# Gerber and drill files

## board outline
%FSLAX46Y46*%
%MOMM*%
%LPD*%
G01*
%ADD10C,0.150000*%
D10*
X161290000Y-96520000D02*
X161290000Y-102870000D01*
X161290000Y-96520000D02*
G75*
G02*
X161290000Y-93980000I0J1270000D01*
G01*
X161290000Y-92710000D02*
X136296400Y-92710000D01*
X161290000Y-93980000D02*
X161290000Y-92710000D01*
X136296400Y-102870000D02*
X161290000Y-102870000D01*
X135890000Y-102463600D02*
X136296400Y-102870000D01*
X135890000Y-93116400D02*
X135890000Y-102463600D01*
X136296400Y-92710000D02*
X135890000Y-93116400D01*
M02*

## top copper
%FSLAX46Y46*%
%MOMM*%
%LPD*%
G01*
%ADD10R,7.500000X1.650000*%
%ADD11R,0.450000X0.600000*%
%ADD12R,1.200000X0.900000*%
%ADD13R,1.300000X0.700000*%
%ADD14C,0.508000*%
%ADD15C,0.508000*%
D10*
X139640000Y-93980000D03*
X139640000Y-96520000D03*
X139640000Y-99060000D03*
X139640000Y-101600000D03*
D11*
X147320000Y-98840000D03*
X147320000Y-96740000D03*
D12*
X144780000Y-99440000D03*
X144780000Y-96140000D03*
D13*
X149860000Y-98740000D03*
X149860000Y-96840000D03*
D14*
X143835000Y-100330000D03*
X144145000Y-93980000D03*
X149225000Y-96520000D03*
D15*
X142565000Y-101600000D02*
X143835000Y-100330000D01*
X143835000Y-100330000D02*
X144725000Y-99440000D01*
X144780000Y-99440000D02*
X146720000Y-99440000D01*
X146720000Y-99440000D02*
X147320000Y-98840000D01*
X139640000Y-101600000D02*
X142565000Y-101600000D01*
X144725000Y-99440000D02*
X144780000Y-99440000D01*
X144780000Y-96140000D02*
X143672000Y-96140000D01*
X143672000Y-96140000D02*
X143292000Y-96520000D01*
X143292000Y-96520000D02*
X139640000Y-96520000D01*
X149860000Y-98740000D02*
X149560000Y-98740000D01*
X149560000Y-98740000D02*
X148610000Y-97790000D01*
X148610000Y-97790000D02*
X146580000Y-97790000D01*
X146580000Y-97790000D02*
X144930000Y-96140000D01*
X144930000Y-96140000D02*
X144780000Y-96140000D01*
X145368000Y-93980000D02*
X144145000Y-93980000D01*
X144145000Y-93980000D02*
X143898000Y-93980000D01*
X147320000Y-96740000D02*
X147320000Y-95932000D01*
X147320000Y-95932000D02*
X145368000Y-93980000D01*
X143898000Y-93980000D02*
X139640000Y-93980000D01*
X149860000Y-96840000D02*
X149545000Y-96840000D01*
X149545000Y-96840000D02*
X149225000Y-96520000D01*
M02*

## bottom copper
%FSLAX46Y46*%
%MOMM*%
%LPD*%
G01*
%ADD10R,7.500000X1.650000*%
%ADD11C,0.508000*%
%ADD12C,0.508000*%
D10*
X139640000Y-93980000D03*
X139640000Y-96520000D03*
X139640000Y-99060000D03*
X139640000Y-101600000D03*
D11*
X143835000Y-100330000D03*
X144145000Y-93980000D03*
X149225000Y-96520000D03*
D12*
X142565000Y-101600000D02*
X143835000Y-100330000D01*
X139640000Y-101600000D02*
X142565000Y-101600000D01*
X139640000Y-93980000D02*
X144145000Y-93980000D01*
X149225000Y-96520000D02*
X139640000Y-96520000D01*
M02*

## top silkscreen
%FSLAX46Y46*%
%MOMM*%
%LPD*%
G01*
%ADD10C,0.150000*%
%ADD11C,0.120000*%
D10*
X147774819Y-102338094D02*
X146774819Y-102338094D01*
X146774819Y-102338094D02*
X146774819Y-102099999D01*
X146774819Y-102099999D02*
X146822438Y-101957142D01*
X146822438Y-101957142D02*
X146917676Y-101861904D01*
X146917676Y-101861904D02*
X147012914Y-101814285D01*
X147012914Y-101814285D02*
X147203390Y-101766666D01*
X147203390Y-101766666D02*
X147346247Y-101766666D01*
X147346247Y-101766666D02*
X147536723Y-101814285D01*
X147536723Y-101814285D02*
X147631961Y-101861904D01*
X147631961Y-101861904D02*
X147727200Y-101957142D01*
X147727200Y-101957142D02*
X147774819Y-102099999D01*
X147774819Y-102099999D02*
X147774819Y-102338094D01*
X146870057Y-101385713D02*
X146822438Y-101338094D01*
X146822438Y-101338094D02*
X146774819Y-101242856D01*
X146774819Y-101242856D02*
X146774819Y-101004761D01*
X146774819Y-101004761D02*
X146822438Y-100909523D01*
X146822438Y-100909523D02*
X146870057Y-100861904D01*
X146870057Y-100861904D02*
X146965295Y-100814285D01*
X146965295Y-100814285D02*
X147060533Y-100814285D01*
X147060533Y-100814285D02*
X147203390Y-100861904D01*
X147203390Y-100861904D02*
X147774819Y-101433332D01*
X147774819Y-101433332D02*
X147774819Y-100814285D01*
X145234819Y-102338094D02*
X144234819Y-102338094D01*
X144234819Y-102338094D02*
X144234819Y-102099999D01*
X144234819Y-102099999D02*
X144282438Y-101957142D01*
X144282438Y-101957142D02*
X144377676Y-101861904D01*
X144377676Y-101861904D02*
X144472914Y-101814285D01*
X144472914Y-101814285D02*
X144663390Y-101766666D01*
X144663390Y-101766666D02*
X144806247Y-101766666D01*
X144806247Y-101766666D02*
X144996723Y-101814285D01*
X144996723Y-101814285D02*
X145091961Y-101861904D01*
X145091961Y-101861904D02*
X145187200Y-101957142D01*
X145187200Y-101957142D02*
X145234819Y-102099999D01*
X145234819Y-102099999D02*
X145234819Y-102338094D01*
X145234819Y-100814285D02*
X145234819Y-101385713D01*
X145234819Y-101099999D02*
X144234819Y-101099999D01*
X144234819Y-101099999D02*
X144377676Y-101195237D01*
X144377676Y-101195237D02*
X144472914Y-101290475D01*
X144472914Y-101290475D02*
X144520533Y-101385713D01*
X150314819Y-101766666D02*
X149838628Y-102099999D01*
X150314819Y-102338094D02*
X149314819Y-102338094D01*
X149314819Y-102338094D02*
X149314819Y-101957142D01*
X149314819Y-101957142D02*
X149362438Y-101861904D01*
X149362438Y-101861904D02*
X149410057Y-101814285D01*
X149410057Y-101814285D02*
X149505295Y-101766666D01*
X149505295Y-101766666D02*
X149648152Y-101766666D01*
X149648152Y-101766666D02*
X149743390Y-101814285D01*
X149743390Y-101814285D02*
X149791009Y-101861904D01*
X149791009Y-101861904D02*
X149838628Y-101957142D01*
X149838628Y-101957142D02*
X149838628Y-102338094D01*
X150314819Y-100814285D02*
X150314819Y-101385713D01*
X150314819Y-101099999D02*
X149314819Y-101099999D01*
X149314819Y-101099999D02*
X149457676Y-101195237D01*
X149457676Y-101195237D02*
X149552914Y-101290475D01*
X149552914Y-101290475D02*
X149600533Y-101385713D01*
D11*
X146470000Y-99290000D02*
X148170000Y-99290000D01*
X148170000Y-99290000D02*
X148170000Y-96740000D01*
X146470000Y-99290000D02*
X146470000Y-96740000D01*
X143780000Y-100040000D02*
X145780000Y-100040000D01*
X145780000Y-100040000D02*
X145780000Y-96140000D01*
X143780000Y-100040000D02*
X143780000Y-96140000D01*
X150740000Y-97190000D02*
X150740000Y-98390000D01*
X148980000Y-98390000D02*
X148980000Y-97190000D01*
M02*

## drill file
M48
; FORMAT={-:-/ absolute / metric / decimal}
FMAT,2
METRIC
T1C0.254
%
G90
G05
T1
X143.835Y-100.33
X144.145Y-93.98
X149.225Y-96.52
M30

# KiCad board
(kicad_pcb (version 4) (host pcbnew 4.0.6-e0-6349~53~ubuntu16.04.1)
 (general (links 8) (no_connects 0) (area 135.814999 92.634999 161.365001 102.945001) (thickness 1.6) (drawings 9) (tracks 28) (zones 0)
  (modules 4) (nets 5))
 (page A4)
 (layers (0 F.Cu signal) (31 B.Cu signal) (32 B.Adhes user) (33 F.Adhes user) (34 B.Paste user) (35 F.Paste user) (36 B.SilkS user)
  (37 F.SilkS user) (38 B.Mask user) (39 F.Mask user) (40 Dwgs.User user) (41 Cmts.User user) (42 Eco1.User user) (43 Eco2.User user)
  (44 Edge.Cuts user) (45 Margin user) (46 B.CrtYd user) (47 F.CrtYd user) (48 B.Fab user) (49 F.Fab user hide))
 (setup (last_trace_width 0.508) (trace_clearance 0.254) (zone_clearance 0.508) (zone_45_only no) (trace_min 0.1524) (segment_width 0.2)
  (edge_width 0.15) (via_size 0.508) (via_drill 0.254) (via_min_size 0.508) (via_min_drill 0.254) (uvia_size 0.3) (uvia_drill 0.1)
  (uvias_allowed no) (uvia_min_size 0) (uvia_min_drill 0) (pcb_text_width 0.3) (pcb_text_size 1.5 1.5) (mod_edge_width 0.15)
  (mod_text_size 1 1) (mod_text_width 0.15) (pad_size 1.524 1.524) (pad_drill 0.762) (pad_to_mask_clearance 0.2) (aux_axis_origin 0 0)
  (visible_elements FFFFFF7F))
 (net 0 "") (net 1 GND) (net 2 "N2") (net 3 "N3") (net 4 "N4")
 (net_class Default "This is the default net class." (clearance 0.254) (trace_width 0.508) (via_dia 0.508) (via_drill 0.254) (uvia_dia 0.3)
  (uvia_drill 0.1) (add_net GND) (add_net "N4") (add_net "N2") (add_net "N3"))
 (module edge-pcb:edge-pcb (layer F.Cu) (at 135.89 97.79 270)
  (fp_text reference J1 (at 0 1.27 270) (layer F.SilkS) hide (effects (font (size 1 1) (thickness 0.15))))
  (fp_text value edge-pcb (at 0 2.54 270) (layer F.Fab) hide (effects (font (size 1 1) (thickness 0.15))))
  (pad 1 smd rect (at -3.81 -3.75 270) (size 1.65 7.5) (layers F.Cu F.Paste F.Mask) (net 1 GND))
  (pad 2 smd rect (at -3.81 -3.75 270) (size 1.65 7.5) (layers B.Cu B.Paste B.Mask) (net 1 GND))
  (pad 3 smd rect (at -1.27 -3.75 270) (size 1.65 7.5) (layers F.Cu F.Paste F.Mask) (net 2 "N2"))
  (pad 4 smd rect (at -1.27 -3.75 270) (size 1.65 7.5) (layers B.Cu B.Paste B.Mask) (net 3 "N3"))
  (pad 5 smd rect (at 1.27 -3.75 270) (size 1.65 7.5) (layers F.Cu F.Paste F.Mask))
  (pad 6 smd rect (at 1.27 -3.75 270) (size 1.65 7.5) (layers B.Cu B.Paste B.Mask))
  (pad 7 smd rect (at 3.81 -3.75 270) (size 1.65 7.5) (layers F.Cu F.Paste F.Mask) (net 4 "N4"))
  (pad 8 smd rect (at 3.81 -3.75 270) (size 1.65 7.5) (layers B.Cu B.Paste B.Mask) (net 4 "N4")))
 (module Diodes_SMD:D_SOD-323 (layer F.Cu) (at 147.32 97.79 90)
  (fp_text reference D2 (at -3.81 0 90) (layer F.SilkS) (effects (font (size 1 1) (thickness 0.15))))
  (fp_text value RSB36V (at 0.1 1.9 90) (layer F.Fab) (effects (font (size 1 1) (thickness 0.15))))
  (fp_line (start -1.5 -0.85) (end -1.5 0.85) (layer F.SilkS) (width 0.12))
  (fp_line (start -1.5 0.85) (end 1.05 0.85) (layer F.SilkS) (width 0.12))
  (fp_line (start -1.5 -0.85) (end 1.05 -0.85) (layer F.SilkS) (width 0.12))
  (pad 1 smd rect (at -1.05 0 90) (size 0.6 0.45) (layers F.Cu F.Paste F.Mask) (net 4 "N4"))
  (pad 2 smd rect (at 1.05 0 90) (size 0.6 0.45) (layers F.Cu F.Paste F.Mask) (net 1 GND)))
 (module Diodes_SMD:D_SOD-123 (layer F.Cu) (at 144.78 97.79 90)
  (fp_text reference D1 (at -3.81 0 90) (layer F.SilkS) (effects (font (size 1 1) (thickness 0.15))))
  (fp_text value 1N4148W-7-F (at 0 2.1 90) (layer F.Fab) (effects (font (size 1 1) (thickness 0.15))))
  (fp_line (start -2.25 -1) (end -2.25 1) (layer F.SilkS) (width 0.12))
  (fp_line (start -2.25 1) (end 1.65 1) (layer F.SilkS) (width 0.12))
  (fp_line (start -2.25 -1) (end 1.65 -1) (layer F.SilkS) (width 0.12))
  (pad 1 smd rect (at -1.65 0 90) (size 0.9 1.2) (layers F.Cu F.Paste F.Mask) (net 4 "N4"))
  (pad 2 smd rect (at 1.65 0 90) (size 0.9 1.2) (layers F.Cu F.Paste F.Mask) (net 2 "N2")))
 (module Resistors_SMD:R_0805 (layer F.Cu) (at 149.86 97.79 90)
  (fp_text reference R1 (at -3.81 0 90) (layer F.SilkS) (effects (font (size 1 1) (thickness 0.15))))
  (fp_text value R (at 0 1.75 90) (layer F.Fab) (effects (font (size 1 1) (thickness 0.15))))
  (fp_line (start 0.6 0.88) (end -0.6 0.88) (layer F.SilkS) (width 0.12))
  (fp_line (start -0.6 -0.88) (end 0.6 -0.88) (layer F.SilkS) (width 0.12))
  (pad 1 smd rect (at -0.95 0 90) (size 0.7 1.3) (layers F.Cu F.Paste F.Mask) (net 2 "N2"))
  (pad 2 smd rect (at 0.95 0 90) (size 0.7 1.3) (layers F.Cu F.Paste F.Mask) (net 3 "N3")))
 (gr_line (start 161.29 96.52) (end 161.29 102.87) (layer Edge.Cuts) (width 0.15))
 (gr_arc (start 161.29 95.25) (end 161.29 96.52) (angle 180) (layer Edge.Cuts) (width 0.15))
 (gr_line (start 161.29 92.71) (end 136.2964 92.71) (layer Edge.Cuts) (width 0.15))
 (gr_line (start 161.29 93.98) (end 161.29 92.71) (layer Edge.Cuts) (width 0.15))
 (gr_line (start 136.2964 102.87) (end 161.29 102.87) (layer Edge.Cuts) (width 0.15))
 (gr_line (start 135.89 102.4636) (end 136.2964 102.87) (layer Edge.Cuts) (width 0.15))
 (gr_line (start 135.89 93.1164) (end 135.89 102.4636) (layer Edge.Cuts) (width 0.15))
 (gr_line (start 136.2964 92.71) (end 135.89 93.1164) (layer Edge.Cuts) (width 0.15))
 (segment (start 142.565 101.6) (end 143.835 100.33) (width 0.508) (layer F.Cu) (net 4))
 (segment (start 142.565 101.6) (end 143.835 100.33) (width 0.508) (layer B.Cu) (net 4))
 (segment (start 143.835 100.33) (end 144.725 99.44) (width 0.508) (layer F.Cu) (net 4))
 (segment (start 139.64 101.6) (end 142.565 101.6) (width 0.508) (layer B.Cu) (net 4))
 (via (at 143.835 100.33) (size 0.508) (drill 0.254) (layers F.Cu B.Cu) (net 4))
 (segment (start 144.78 99.44) (end 146.72 99.44) (width 0.508) (layer F.Cu) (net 4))
 (segment (start 146.72 99.44) (end 147.32 98.84) (width 0.508) (layer F.Cu) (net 4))
 (segment (start 139.64 101.6) (end 142.565 101.6) (width 0.508) (layer F.Cu) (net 4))
 (segment (start 144.725 99.44) (end 144.78 99.44) (width 0.508) (layer F.Cu) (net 4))
 (segment (start 144.78 96.14) (end 143.672 96.14) (width 0.508) (layer F.Cu) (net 2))
 (segment (start 143.672 96.14) (end 143.292 96.52) (width 0.508) (layer F.Cu) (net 2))
 (segment (start 143.292 96.52) (end 139.64 96.52) (width 0.508) (layer F.Cu) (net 2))
 (segment (start 149.86 98.74) (end 149.56 98.74) (width 0.508) (layer F.Cu) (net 2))
 (segment (start 149.56 98.74) (end 148.61 97.79) (width 0.508) (layer F.Cu) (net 2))
 (segment (start 148.61 97.79) (end 146.58 97.79) (width 0.508) (layer F.Cu) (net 2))
 (segment (start 146.58 97.79) (end 144.93 96.14) (width 0.508) (layer F.Cu) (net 2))
 (segment (start 144.93 96.14) (end 144.78 96.14) (width 0.508) (layer F.Cu) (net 2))
 (segment (start 145.368 93.98) (end 144.145 93.98) (width 0.508) (layer F.Cu) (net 1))
 (segment (start 144.145 93.98) (end 143.898 93.98) (width 0.508) (layer F.Cu) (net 1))
 (segment (start 139.64 93.98) (end 144.145 93.98) (width 0.508) (layer B.Cu) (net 1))
 (via (at 144.145 93.98) (size 0.508) (drill 0.254) (layers F.Cu B.Cu) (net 1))
 (segment (start 147.32 96.74) (end 147.32 95.932) (width 0.508) (layer F.Cu) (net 1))
 (segment (start 147.32 95.932) (end 145.368 93.98) (width 0.508) (layer F.Cu) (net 1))
 (segment (start 143.898 93.98) (end 139.64 93.98) (width 0.508) (layer F.Cu) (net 1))
 (segment (start 149.225 96.52) (end 139.64 96.52) (width 0.508) (layer B.Cu) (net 3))
 (segment (start 149.86 96.84) (end 149.545 96.84) (width 0.508) (layer F.Cu) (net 3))
 (segment (start 149.545 96.84) (end 149.225 96.52) (width 0.508) (layer F.Cu) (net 3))
 (via (at 149.225 96.52) (size 0.508) (drill 0.254) (layers F.Cu B.Cu) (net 3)))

